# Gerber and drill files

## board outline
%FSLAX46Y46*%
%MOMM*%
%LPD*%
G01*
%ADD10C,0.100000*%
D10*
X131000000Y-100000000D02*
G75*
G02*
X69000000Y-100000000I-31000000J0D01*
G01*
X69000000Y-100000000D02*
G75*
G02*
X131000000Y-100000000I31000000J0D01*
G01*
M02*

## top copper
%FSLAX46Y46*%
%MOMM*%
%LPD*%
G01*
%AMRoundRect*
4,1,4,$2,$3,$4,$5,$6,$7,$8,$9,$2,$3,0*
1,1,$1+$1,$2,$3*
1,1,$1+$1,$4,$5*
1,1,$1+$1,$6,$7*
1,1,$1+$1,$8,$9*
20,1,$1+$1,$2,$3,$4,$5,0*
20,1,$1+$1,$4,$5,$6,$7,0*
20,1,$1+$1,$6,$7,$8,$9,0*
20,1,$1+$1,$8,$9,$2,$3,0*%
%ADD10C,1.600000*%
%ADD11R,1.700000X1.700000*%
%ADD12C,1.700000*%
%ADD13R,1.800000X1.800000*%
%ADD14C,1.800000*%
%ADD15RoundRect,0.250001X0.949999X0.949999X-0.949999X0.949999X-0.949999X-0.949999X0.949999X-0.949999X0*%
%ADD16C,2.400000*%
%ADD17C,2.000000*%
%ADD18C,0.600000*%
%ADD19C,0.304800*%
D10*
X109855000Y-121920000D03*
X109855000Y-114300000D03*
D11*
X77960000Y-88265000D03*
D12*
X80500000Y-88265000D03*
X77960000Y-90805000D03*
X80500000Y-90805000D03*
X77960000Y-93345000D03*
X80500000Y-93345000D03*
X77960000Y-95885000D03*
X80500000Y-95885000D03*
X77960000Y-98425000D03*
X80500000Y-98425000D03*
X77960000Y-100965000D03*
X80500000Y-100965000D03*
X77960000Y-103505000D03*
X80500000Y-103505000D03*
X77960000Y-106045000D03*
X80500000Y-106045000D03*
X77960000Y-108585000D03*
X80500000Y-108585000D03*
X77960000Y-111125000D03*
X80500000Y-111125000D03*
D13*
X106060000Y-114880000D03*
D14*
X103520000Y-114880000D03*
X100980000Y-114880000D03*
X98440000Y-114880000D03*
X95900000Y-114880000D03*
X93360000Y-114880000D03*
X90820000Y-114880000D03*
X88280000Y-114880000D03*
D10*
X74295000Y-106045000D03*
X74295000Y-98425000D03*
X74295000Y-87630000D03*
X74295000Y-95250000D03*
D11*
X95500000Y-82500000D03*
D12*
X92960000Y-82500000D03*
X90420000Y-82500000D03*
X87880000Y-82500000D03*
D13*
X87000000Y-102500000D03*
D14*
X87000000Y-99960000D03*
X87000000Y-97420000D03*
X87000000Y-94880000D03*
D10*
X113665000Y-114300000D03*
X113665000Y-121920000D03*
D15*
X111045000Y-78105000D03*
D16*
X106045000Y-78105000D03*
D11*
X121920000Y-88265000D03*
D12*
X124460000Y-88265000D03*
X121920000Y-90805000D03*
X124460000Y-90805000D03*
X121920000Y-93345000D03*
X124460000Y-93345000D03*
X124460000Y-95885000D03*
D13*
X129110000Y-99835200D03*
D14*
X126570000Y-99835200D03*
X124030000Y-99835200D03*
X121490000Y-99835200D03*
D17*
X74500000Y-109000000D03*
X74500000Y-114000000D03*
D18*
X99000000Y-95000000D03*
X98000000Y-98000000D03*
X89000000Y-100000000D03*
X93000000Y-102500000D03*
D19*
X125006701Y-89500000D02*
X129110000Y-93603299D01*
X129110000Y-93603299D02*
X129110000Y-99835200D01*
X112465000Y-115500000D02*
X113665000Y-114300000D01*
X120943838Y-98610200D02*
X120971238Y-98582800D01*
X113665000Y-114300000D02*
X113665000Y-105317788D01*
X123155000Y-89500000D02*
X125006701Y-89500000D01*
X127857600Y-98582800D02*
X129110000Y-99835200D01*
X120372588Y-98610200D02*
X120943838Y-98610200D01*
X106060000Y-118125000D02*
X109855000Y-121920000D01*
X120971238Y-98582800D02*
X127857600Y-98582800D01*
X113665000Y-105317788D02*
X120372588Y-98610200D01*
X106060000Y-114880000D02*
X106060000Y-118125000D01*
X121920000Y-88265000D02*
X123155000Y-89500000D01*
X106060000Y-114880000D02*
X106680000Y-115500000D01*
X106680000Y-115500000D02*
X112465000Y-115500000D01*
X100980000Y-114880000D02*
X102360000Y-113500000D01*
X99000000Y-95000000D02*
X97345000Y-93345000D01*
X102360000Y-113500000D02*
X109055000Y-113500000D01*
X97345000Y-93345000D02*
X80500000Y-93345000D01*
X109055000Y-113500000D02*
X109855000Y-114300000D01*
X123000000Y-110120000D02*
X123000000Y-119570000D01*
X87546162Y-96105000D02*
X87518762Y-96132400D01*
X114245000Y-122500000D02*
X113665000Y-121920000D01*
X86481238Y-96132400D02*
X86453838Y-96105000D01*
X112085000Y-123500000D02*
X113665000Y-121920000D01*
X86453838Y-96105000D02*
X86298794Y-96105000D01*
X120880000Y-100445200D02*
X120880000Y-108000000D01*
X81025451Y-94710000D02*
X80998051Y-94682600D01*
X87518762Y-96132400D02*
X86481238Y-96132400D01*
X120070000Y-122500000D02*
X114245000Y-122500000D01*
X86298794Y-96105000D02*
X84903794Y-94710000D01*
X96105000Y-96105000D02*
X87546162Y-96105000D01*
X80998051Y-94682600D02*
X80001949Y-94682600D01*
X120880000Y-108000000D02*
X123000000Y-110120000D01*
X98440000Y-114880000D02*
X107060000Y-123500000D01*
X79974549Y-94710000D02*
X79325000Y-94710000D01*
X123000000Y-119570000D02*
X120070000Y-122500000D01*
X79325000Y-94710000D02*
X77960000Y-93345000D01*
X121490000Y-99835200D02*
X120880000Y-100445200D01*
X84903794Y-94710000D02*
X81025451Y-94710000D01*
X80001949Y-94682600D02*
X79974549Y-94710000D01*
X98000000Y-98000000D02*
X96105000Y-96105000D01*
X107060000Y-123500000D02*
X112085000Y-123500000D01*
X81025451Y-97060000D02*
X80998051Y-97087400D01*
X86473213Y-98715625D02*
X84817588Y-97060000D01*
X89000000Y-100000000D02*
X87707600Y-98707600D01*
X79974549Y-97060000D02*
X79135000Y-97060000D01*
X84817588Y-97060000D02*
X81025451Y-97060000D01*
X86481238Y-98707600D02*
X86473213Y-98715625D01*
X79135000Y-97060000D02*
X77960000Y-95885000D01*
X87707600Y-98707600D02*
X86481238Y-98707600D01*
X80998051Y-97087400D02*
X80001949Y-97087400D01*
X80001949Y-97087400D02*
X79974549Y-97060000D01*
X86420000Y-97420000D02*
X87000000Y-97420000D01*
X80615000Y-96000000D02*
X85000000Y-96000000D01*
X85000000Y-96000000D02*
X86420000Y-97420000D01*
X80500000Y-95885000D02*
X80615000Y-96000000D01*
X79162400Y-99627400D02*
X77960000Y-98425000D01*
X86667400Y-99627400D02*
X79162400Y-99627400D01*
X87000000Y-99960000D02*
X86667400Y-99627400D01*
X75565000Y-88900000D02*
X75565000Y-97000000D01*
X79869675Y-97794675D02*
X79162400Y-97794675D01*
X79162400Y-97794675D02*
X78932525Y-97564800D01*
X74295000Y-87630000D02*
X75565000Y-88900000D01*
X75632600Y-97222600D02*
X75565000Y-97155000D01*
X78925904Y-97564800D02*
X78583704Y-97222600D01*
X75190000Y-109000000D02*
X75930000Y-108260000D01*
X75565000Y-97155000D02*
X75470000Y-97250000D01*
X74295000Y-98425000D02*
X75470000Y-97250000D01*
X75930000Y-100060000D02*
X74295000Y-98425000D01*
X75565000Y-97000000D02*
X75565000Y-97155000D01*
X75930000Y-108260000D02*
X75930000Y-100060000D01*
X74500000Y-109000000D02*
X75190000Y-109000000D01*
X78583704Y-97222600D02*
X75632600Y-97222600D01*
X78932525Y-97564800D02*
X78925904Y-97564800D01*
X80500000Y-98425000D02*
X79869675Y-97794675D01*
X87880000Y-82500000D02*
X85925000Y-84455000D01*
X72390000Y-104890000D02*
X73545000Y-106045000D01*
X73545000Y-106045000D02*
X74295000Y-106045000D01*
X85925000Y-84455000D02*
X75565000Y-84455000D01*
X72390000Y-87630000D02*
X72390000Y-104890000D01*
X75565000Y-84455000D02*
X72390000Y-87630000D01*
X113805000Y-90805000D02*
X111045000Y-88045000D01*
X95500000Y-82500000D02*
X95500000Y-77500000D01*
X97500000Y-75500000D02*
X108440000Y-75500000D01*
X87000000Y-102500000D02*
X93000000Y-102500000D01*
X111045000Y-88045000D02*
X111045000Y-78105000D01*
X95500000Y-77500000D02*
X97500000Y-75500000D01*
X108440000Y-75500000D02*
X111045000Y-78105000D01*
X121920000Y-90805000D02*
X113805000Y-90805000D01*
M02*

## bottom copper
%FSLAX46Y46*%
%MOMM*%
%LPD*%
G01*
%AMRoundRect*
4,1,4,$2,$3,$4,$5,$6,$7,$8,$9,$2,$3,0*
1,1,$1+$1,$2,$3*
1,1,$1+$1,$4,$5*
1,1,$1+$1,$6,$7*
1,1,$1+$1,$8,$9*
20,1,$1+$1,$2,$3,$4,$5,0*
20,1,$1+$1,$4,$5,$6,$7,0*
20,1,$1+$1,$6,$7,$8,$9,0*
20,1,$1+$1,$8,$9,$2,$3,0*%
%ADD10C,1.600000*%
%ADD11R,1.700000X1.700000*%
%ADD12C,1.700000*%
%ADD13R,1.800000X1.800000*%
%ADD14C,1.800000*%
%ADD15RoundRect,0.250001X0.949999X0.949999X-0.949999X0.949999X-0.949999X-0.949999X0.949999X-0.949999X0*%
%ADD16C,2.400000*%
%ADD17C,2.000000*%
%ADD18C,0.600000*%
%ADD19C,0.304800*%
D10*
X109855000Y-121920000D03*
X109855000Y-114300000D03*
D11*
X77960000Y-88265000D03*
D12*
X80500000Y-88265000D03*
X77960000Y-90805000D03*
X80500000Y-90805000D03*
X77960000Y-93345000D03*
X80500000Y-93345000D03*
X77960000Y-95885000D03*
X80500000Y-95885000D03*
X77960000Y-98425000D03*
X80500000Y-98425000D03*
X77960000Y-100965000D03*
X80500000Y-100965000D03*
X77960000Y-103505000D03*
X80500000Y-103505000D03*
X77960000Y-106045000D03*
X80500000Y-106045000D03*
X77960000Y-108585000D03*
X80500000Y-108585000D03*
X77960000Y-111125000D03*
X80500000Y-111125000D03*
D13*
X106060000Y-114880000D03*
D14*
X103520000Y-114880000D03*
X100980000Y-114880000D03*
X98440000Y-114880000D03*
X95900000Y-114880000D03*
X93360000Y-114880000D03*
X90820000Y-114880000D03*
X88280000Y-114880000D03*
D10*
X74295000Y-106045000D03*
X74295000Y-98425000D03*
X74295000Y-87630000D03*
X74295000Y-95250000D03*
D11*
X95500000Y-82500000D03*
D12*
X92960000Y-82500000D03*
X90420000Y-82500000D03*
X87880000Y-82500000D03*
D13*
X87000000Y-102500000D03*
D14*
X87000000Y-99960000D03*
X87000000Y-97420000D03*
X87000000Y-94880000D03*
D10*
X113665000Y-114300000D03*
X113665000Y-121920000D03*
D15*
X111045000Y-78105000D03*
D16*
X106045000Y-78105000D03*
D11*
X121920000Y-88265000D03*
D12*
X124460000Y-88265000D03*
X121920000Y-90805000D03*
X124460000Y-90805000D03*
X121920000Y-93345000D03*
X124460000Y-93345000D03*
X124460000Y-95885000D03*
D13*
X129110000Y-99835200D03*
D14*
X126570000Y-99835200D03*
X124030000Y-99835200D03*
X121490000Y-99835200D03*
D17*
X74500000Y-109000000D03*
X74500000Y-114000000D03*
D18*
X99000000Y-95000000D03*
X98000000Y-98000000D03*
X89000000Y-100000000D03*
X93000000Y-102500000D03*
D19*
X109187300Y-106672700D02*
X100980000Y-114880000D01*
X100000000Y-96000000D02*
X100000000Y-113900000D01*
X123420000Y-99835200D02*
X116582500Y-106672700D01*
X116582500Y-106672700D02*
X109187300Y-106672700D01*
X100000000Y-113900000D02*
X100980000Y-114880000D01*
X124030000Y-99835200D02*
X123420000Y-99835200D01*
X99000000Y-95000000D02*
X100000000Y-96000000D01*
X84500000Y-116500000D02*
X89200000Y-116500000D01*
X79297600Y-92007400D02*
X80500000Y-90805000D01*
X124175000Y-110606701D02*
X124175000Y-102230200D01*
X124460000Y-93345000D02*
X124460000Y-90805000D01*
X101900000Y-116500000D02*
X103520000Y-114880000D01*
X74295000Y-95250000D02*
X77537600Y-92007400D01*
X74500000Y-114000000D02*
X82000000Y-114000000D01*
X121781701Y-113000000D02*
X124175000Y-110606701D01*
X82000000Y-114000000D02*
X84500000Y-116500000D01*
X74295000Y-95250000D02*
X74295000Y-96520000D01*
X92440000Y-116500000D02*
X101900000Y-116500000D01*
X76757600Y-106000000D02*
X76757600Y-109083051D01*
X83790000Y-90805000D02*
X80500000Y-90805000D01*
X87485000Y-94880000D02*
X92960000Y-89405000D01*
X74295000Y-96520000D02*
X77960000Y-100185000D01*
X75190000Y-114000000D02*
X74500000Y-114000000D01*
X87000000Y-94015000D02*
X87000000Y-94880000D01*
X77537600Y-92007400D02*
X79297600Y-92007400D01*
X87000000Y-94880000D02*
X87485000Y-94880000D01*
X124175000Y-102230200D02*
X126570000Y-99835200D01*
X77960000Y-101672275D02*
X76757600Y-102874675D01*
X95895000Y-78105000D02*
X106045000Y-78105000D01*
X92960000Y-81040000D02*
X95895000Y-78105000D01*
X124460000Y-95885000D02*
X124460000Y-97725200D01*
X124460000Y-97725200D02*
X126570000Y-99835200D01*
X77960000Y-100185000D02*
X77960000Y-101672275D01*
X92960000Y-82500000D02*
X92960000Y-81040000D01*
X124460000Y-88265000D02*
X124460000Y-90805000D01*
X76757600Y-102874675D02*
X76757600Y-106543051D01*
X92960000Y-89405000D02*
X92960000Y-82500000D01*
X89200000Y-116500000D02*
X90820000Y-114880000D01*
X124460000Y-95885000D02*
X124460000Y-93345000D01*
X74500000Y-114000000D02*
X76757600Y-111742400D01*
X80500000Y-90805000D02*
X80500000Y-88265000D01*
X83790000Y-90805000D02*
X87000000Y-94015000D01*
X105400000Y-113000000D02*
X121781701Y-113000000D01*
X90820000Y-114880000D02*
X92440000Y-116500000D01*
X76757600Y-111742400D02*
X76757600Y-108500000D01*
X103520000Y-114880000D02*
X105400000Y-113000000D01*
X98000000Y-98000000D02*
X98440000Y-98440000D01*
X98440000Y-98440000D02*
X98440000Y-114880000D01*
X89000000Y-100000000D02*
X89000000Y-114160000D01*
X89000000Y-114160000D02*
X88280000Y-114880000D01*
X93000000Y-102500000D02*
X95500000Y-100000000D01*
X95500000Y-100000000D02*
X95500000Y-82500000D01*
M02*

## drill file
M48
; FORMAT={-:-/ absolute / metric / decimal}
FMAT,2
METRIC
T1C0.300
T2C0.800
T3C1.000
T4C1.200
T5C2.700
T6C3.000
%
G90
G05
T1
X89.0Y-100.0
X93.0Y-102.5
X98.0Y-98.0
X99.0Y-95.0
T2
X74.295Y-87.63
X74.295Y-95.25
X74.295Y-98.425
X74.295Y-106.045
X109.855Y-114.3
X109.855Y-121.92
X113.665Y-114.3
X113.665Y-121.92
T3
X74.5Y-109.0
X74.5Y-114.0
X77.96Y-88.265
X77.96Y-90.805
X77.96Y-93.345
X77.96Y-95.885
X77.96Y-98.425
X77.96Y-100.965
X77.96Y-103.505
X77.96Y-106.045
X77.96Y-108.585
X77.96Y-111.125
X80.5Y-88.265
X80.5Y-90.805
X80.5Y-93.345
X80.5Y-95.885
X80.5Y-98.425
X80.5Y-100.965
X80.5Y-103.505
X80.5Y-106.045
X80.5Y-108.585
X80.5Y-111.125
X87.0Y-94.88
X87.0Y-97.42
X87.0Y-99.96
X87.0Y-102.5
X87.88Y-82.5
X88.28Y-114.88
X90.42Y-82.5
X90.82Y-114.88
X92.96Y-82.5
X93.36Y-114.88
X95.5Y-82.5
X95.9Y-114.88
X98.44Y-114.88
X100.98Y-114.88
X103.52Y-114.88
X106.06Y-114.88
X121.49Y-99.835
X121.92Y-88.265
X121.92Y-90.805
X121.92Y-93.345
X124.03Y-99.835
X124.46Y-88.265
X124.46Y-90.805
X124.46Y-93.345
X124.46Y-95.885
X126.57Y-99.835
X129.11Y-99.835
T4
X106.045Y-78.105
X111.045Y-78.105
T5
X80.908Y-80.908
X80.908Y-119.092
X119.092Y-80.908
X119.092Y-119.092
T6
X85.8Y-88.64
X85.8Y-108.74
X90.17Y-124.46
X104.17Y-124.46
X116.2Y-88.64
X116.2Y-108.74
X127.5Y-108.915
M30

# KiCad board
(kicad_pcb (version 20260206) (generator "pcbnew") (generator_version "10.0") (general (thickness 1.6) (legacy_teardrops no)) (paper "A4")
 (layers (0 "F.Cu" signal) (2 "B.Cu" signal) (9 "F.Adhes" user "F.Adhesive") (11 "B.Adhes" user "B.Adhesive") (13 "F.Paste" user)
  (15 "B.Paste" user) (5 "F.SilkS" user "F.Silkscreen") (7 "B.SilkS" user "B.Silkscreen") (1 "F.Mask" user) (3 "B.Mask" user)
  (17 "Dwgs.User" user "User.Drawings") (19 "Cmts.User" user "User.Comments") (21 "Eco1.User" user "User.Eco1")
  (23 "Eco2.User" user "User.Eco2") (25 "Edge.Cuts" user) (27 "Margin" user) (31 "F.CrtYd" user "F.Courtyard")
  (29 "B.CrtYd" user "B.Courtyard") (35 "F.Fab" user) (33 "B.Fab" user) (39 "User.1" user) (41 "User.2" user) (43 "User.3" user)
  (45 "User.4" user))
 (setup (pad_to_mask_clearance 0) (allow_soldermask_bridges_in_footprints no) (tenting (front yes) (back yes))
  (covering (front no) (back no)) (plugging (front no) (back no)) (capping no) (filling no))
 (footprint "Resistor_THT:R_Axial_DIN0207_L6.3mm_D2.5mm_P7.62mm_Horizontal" (layer "F.Cu") (at 109.855 121.92 90)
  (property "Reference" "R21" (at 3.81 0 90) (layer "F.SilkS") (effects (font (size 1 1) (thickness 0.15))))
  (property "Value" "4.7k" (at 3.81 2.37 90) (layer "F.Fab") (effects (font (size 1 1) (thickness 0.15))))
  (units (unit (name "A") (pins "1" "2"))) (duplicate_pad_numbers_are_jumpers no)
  (pad "1" thru_hole circle (at 0 0 90) (size 1.6 1.6) (drill 0.8) (layers "*.Cu" "*.Mask") (remove_unused_layers no) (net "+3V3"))
  (pad "2" thru_hole circle (at 7.62 0 90) (size 1.6 1.6) (drill 0.8) (layers "*.Cu" "*.Mask") (remove_unused_layers no) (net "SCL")))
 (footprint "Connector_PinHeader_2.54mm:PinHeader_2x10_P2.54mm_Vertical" (layer "F.Cu") (at 77.96 88.265)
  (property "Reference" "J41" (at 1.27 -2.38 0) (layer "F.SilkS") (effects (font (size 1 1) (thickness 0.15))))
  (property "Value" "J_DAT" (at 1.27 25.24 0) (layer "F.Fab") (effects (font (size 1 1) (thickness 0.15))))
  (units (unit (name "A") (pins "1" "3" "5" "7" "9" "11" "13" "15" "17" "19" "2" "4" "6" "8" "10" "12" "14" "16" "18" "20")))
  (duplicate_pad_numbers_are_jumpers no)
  (pad "1" thru_hole rect (at 0 0) (size 1.7 1.7) (drill 1) (layers "*.Cu" "*.Mask") (remove_unused_layers no)
   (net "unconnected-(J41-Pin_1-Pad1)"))
  (pad "2" thru_hole circle (at 2.54 0) (size 1.7 1.7) (drill 1) (layers "*.Cu" "*.Mask") (remove_unused_layers no) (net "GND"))
  (pad "3" thru_hole circle (at 0 2.54) (size 1.7 1.7) (drill 1) (layers "*.Cu" "*.Mask") (remove_unused_layers no)
   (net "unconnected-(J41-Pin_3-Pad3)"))
  (pad "4" thru_hole circle (at 2.54 2.54) (size 1.7 1.7) (drill 1) (layers "*.Cu" "*.Mask") (remove_unused_layers no) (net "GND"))
  (pad "5" thru_hole circle (at 0 5.08) (size 1.7 1.7) (drill 1) (layers "*.Cu" "*.Mask") (remove_unused_layers no) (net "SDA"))
  (pad "6" thru_hole circle (at 2.54 5.08) (size 1.7 1.7) (drill 1) (layers "*.Cu" "*.Mask") (remove_unused_layers no) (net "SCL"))
  (pad "7" thru_hole circle (at 0 7.62) (size 1.7 1.7) (drill 1) (layers "*.Cu" "*.Mask") (remove_unused_layers no) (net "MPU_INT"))
  (pad "8" thru_hole circle (at 2.54 7.62) (size 1.7 1.7) (drill 1) (layers "*.Cu" "*.Mask") (remove_unused_layers no) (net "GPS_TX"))
  (pad "9" thru_hole circle (at 0 10.16) (size 1.7 1.7) (drill 1) (layers "*.Cu" "*.Mask") (remove_unused_layers no) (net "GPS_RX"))
  (pad "10" thru_hole circle (at 2.54 10.16) (size 1.7 1.7) (drill 1) (layers "*.Cu" "*.Mask") (remove_unused_layers no) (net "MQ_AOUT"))
  (pad "11" thru_hole circle (at 0 12.7) (size 1.7 1.7) (drill 1) (layers "*.Cu" "*.Mask") (remove_unused_layers no) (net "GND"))
  (pad "12" thru_hole circle (at 2.54 12.7) (size 1.7 1.7) (drill 1) (layers "*.Cu" "*.Mask") (remove_unused_layers no)
   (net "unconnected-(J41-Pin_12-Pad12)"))
  (pad "13" thru_hole circle (at 0 15.24) (size 1.7 1.7) (drill 1) (layers "*.Cu" "*.Mask") (remove_unused_layers no)
   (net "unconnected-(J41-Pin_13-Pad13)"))
  (pad "14" thru_hole circle (at 2.54 15.24) (size 1.7 1.7) (drill 1) (layers "*.Cu" "*.Mask") (remove_unused_layers no)
   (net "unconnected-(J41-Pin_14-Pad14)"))
  (pad "15" thru_hole circle (at 0 17.78) (size 1.7 1.7) (drill 1) (layers "*.Cu" "*.Mask") (remove_unused_layers no)
   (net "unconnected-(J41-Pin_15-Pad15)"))
  (pad "16" thru_hole circle (at 2.54 17.78) (size 1.7 1.7) (drill 1) (layers "*.Cu" "*.Mask") (remove_unused_layers no)
   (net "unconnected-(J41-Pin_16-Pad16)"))
  (pad "17" thru_hole circle (at 0 20.32) (size 1.7 1.7) (drill 1) (layers "*.Cu" "*.Mask") (remove_unused_layers no)
   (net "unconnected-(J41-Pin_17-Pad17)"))
  (pad "18" thru_hole circle (at 2.54 20.32) (size 1.7 1.7) (drill 1) (layers "*.Cu" "*.Mask") (remove_unused_layers no)
   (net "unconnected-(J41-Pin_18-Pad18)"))
  (pad "19" thru_hole circle (at 0 22.86) (size 1.7 1.7) (drill 1) (layers "*.Cu" "*.Mask") (remove_unused_layers no)
   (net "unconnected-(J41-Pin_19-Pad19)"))
  (pad "20" thru_hole circle (at 2.54 22.86) (size 1.7 1.7) (drill 1) (layers "*.Cu" "*.Mask") (remove_unused_layers no)
   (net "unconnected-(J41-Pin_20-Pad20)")))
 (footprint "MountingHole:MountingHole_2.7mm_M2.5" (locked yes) (layer "F.Cu") (at 119.092 119.092)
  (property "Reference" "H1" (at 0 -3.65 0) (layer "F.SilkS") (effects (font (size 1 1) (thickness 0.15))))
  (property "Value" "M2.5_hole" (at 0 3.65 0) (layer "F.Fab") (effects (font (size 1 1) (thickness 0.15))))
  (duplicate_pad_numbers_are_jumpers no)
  (pad "" np_thru_hole circle (at 0 0) (size 2.7 2.7) (drill 2.7) (layers "*.Cu" "*.Mask")))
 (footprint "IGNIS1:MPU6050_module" (layer "F.Cu") (at 97.17 119.96 -90)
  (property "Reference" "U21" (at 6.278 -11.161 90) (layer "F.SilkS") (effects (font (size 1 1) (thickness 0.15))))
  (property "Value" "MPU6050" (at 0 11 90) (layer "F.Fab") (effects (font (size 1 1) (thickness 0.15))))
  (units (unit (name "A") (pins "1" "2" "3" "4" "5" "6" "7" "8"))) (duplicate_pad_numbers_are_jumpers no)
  (pad "" np_thru_hole circle (at 4.5 -7 270) (size 3 3) (drill 3) (layers "*.Cu" "*.Mask"))
  (pad "" np_thru_hole circle (at 4.5 7 270) (size 3 3) (drill 3) (layers "*.Cu" "*.Mask"))
  (pad "1" thru_hole rect (at -5.08 -8.89 270) (size 1.8 1.8) (drill 1) (layers "*.Cu" "*.Mask") (remove_unused_layers no) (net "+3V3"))
  (pad "2" thru_hole circle (at -5.08 -6.35 270) (size 1.8 1.8) (drill 1) (layers "*.Cu" "*.Mask") (remove_unused_layers no) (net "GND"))
  (pad "3" thru_hole circle (at -5.08 -3.81 270) (size 1.8 1.8) (drill 1) (layers "*.Cu" "*.Mask") (remove_unused_layers no) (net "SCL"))
  (pad "4" thru_hole circle (at -5.08 -1.27 270) (size 1.8 1.8) (drill 1) (layers "*.Cu" "*.Mask") (remove_unused_layers no) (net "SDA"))
  (pad "5" thru_hole circle (at -5.08 1.27 270) (size 1.8 1.8) (drill 1) (layers "*.Cu" "*.Mask") (remove_unused_layers no)
   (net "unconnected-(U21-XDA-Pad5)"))
  (pad "6" thru_hole circle (at -5.08 3.81 270) (size 1.8 1.8) (drill 1) (layers "*.Cu" "*.Mask") (remove_unused_layers no)
   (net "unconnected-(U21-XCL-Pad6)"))
  (pad "7" thru_hole circle (at -5.08 6.35 270) (size 1.8 1.8) (drill 1) (layers "*.Cu" "*.Mask") (remove_unused_layers no) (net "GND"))
  (pad "8" thru_hole circle (at -5.08 8.89 270) (size 1.8 1.8) (drill 1) (layers "*.Cu" "*.Mask") (remove_unused_layers no) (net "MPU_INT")))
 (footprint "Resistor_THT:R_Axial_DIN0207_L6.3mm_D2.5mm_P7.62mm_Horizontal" (layer "F.Cu") (at 74.295 106.045 90)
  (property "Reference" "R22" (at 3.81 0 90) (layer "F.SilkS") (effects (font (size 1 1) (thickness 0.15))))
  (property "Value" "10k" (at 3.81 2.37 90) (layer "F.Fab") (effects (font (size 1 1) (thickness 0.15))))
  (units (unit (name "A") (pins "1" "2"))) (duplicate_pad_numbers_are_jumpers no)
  (pad "1" thru_hole circle (at 0 0 90) (size 1.6 1.6) (drill 0.8) (layers "*.Cu" "*.Mask") (remove_unused_layers no) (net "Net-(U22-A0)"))
  (pad "2" thru_hole circle (at 7.62 0 90) (size 1.6 1.6) (drill 0.8) (layers "*.Cu" "*.Mask") (remove_unused_layers no) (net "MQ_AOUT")))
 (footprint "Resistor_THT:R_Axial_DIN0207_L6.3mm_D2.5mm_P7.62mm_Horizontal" (layer "F.Cu") (at 74.295 87.63 -90)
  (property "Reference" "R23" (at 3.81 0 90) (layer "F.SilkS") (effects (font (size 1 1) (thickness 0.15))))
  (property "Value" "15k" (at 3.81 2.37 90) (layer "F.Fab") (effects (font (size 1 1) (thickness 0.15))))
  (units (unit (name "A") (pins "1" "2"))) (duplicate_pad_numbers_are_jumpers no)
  (pad "1" thru_hole circle (at 0 0 270) (size 1.6 1.6) (drill 0.8) (layers "*.Cu" "*.Mask") (remove_unused_layers no) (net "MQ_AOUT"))
  (pad "2" thru_hole circle (at 7.62 0 270) (size 1.6 1.6) (drill 0.8) (layers "*.Cu" "*.Mask") (remove_unused_layers no) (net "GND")))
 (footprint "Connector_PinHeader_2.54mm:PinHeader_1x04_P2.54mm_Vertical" (layer "F.Cu") (at 95.5 82.5 -90)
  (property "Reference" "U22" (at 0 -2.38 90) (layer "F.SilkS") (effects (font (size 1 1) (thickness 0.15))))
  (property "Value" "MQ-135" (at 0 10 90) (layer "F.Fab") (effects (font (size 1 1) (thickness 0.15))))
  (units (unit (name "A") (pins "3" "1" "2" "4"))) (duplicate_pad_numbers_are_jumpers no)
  (pad "1" thru_hole rect (at 0 0 270) (size 1.7 1.7) (drill 1) (layers "*.Cu" "*.Mask") (remove_unused_layers no) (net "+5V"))
  (pad "2" thru_hole circle (at 0 2.54 270) (size 1.7 1.7) (drill 1) (layers "*.Cu" "*.Mask") (remove_unused_layers no) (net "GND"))
  (pad "3" thru_hole circle (at 0 5.08 270) (size 1.7 1.7) (drill 1) (layers "*.Cu" "*.Mask") (remove_unused_layers no)
   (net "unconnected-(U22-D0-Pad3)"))
  (pad "4" thru_hole circle (at 0 7.62 270) (size 1.7 1.7) (drill 1) (layers "*.Cu" "*.Mask") (remove_unused_layers no) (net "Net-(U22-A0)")))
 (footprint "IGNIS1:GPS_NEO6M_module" (layer "F.Cu") (at 101 98.69)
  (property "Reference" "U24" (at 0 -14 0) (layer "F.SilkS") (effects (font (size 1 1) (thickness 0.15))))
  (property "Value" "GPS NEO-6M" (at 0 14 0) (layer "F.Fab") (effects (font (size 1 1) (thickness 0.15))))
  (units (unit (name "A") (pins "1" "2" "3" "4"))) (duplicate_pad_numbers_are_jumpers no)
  (pad "" np_thru_hole circle (at -15.2 -10.05) (size 3 3) (drill 3) (layers "*.Cu" "*.Mask"))
  (pad "" np_thru_hole circle (at -15.2 10.05) (size 3 3) (drill 3) (layers "*.Cu" "*.Mask"))
  (pad "" np_thru_hole circle (at 15.2 -10.05) (size 3 3) (drill 3) (layers "*.Cu" "*.Mask"))
  (pad "" np_thru_hole circle (at 15.2 10.05) (size 3 3) (drill 3) (layers "*.Cu" "*.Mask"))
  (pad "1" thru_hole rect (at -14 3.81) (size 1.8 1.8) (drill 1) (layers "*.Cu" "*.Mask") (remove_unused_layers no) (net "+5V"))
  (pad "2" thru_hole circle (at -14 1.27) (size 1.8 1.8) (drill 1) (layers "*.Cu" "*.Mask") (remove_unused_layers no) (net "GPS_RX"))
  (pad "3" thru_hole circle (at -14 -1.27) (size 1.8 1.8) (drill 1) (layers "*.Cu" "*.Mask") (remove_unused_layers no) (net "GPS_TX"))
  (pad "4" thru_hole circle (at -14 -3.81) (size 1.8 1.8) (drill 1) (layers "*.Cu" "*.Mask") (remove_unused_layers no) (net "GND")))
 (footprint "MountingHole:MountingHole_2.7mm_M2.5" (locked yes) (layer "F.Cu") (at 80.908 80.908)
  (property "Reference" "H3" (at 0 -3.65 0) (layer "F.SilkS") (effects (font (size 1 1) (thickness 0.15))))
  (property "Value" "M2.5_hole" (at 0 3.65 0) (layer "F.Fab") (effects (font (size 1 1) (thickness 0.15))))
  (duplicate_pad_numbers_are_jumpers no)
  (pad "" np_thru_hole circle (at 0 0) (size 2.7 2.7) (drill 2.7) (layers "*.Cu" "*.Mask")))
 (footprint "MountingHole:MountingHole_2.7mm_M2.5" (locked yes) (layer "F.Cu") (at 119.092 80.908)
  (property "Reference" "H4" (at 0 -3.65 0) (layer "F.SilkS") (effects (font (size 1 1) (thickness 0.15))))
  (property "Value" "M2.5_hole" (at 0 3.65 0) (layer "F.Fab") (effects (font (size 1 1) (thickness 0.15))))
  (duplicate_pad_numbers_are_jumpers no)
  (pad "" np_thru_hole circle (at 0 0) (size 2.7 2.7) (drill 2.7) (layers "*.Cu" "*.Mask")))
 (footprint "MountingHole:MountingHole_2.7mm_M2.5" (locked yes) (layer "F.Cu") (at 80.908 119.092)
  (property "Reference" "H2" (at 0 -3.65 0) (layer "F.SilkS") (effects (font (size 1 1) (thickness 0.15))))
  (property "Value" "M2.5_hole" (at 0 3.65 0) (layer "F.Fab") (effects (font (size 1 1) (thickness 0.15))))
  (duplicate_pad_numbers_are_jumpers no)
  (pad "" np_thru_hole circle (at 0 0) (size 2.7 2.7) (drill 2.7) (layers "*.Cu" "*.Mask")))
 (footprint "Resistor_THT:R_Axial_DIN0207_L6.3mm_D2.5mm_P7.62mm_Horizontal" (layer "F.Cu") (at 113.665 114.3 -90)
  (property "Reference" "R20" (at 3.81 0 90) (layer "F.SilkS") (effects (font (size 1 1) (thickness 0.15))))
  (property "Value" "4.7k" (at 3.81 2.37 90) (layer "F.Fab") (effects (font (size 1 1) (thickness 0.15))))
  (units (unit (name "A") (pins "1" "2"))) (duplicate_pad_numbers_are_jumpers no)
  (pad "1" thru_hole circle (at 0 0 270) (size 1.6 1.6) (drill 0.8) (layers "*.Cu" "*.Mask") (remove_unused_layers no) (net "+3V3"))
  (pad "2" thru_hole circle (at 7.62 0 270) (size 1.6 1.6) (drill 0.8) (layers "*.Cu" "*.Mask") (remove_unused_layers no) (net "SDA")))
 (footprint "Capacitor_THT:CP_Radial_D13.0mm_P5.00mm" (layer "F.Cu") (at 111.045 78.105 180)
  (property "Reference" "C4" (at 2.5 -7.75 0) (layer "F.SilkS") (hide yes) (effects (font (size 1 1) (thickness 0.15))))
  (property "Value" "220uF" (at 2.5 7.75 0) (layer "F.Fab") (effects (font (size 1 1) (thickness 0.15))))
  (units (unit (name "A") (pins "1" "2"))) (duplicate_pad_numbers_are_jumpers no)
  (pad "1" thru_hole roundrect (at 0 0 180) (size 2.4 2.4) (drill 1.2) (layers "*.Cu" "*.Mask") (remove_unused_layers no)
   (roundrect_rratio 0.104167) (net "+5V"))
  (pad "2" thru_hole circle (at 5 0 180) (size 2.4 2.4) (drill 1.2) (layers "*.Cu" "*.Mask") (remove_unused_layers no) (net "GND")))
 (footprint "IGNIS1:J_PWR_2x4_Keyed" (layer "F.Cu") (at 123.19 92.075)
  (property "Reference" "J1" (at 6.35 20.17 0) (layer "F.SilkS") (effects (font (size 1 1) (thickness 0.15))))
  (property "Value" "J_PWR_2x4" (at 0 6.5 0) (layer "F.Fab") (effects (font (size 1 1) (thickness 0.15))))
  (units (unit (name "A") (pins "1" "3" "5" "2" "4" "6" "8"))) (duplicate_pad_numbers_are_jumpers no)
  (pad "1" thru_hole rect (at -1.27 -3.81) (size 1.7 1.7) (drill 1) (layers "*.Cu" "*.Mask") (remove_unused_layers no) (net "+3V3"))
  (pad "2" thru_hole circle (at 1.27 -3.81) (size 1.7 1.7) (drill 1) (layers "*.Cu" "*.Mask") (remove_unused_layers no) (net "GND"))
  (pad "3" thru_hole circle (at -1.27 -1.27) (size 1.7 1.7) (drill 1) (layers "*.Cu" "*.Mask") (remove_unused_layers no) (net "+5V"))
  (pad "4" thru_hole circle (at 1.27 -1.27) (size 1.7 1.7) (drill 1) (layers "*.Cu" "*.Mask") (remove_unused_layers no) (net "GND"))
  (pad "5" thru_hole circle (at -1.27 1.27) (size 1.7 1.7) (drill 1) (layers "*.Cu" "*.Mask") (remove_unused_layers no)
   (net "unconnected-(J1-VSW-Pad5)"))
  (pad "6" thru_hole circle (at 1.27 1.27) (size 1.7 1.7) (drill 1) (layers "*.Cu" "*.Mask") (remove_unused_layers no) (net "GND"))
  (pad "8" thru_hole circle (at 1.27 3.81) (size 1.7 1.7) (drill 1) (layers "*.Cu" "*.Mask") (remove_unused_layers no) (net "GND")))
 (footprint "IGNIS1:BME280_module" (layer "F.Cu") (at 125.3 104.9152 -90)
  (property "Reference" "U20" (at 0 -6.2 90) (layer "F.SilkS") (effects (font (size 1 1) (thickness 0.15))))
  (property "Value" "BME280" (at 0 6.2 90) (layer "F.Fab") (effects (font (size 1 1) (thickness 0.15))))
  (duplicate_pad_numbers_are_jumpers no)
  (pad "" np_thru_hole circle (at 4 -2.2 270) (size 3 3) (drill 3) (layers "*.Cu" "*.Mask"))
  (pad "1" thru_hole rect (at -5.08 -3.81 270) (size 1.8 1.8) (drill 1) (layers "*.Cu" "*.Mask") (remove_unused_layers no) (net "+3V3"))
  (pad "2" thru_hole circle (at -5.08 -1.27 270) (size 1.8 1.8) (drill 1) (layers "*.Cu" "*.Mask") (remove_unused_layers no) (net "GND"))
  (pad "3" thru_hole circle (at -5.08 1.27 270) (size 1.8 1.8) (drill 1) (layers "*.Cu" "*.Mask") (remove_unused_layers no) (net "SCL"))
  (pad "4" thru_hole circle (at -5.08 3.81 270) (size 1.8 1.8) (drill 1) (layers "*.Cu" "*.Mask") (remove_unused_layers no) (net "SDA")))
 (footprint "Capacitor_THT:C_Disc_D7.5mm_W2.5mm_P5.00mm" (layer "F.Cu") (at 74.5 109 -90)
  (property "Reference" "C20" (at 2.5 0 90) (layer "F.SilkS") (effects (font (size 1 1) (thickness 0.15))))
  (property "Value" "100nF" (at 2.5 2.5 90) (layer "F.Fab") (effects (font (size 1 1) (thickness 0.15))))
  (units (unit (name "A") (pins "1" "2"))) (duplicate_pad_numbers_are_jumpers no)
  (pad "1" thru_hole circle (at 0 0 270) (size 2 2) (drill 1) (layers "*.Cu" "*.Mask") (remove_unused_layers no) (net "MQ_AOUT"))
  (pad "2" thru_hole circle (at 5 0 270) (size 2 2) (drill 1) (layers "*.Cu" "*.Mask") (remove_unused_layers no) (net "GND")))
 (gr_circle (center 100 100) (end 131 100) (stroke (width 0.1) (type solid)) (fill no) (locked yes) (layer "Edge.Cuts"))
 (segment (start 125.006701 89.5) (end 129.11 93.603299) (width 0.3048) (layer "F.Cu") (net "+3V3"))
 (segment (start 129.11 93.603299) (end 129.11 99.8352) (width 0.3048) (layer "F.Cu") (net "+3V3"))
 (segment (start 112.465 115.5) (end 113.665 114.3) (width 0.3048) (layer "F.Cu") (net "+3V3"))
 (segment (start 120.943838 98.6102) (end 120.971238 98.5828) (width 0.3048) (layer "F.Cu") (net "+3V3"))
 (segment (start 113.665 114.3) (end 113.665 105.317788) (width 0.3048) (layer "F.Cu") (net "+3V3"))
 (segment (start 123.155 89.5) (end 125.006701 89.5) (width 0.3048) (layer "F.Cu") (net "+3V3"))
 (segment (start 127.8576 98.5828) (end 129.11 99.8352) (width 0.3048) (layer "F.Cu") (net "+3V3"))
 (segment (start 120.372588 98.6102) (end 120.943838 98.6102) (width 0.3048) (layer "F.Cu") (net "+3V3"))
 (segment (start 106.06 118.125) (end 109.855 121.92) (width 0.3048) (layer "F.Cu") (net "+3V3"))
 (segment (start 120.971238 98.5828) (end 127.8576 98.5828) (width 0.3048) (layer "F.Cu") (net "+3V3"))
 (segment (start 113.665 105.317788) (end 120.372588 98.6102) (width 0.3048) (layer "F.Cu") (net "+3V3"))
 (segment (start 106.06 114.88) (end 106.06 118.125) (width 0.3048) (layer "F.Cu") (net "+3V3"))
 (segment (start 121.92 88.265) (end 123.155 89.5) (width 0.3048) (layer "F.Cu") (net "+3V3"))
 (segment (start 106.06 114.88) (end 106.68 115.5) (width 0.3048) (layer "F.Cu") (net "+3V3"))
 (segment (start 106.68 115.5) (end 112.465 115.5) (width 0.3048) (layer "F.Cu") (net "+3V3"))
 (segment (start 100.98 114.88) (end 102.36 113.5) (width 0.3048) (layer "F.Cu") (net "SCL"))
 (segment (start 99 95) (end 97.345 93.345) (width 0.3048) (layer "F.Cu") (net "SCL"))
 (segment (start 102.36 113.5) (end 109.055 113.5) (width 0.3048) (layer "F.Cu") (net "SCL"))
 (segment (start 97.345 93.345) (end 80.5 93.345) (width 0.3048) (layer "F.Cu") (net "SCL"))
 (segment (start 109.055 113.5) (end 109.855 114.3) (width 0.3048) (layer "F.Cu") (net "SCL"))
 (via (at 99 95) (size 0.6) (drill 0.3) (layers "F.Cu" "B.Cu") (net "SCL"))
 (segment (start 109.1873 106.6727) (end 100.98 114.88) (width 0.3048) (layer "B.Cu") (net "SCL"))
 (segment (start 100 96) (end 100 113.9) (width 0.3048) (layer "B.Cu") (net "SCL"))
 (segment (start 123.42 99.8352) (end 116.5825 106.6727) (width 0.3048) (layer "B.Cu") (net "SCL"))
 (segment (start 116.5825 106.6727) (end 109.1873 106.6727) (width 0.3048) (layer "B.Cu") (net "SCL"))
 (segment (start 100 113.9) (end 100.98 114.88) (width 0.3048) (layer "B.Cu") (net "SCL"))
 (segment (start 124.03 99.8352) (end 123.42 99.8352) (width 0.3048) (layer "B.Cu") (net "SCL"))
 (segment (start 99 95) (end 100 96) (width 0.3048) (layer "B.Cu") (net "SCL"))
 (segment (start 84.5 116.5) (end 89.2 116.5) (width 0.3048) (layer "B.Cu") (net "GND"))
 (segment (start 79.2976 92.0074) (end 80.5 90.805) (width 0.3048) (layer "B.Cu") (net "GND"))
 (segment (start 124.175 110.606701) (end 124.175 102.2302) (width 0.3048) (layer "B.Cu") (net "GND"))
 (segment (start 124.46 93.345) (end 124.46 90.805) (width 0.3048) (layer "B.Cu") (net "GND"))
 (segment (start 101.9 116.5) (end 103.52 114.88) (width 0.3048) (layer "B.Cu") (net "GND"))
 (segment (start 74.295 95.25) (end 77.5376 92.0074) (width 0.3048) (layer "B.Cu") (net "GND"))
 (segment (start 74.5 114) (end 82 114) (width 0.3048) (layer "B.Cu") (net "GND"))
 (segment (start 121.781701 113) (end 124.175 110.606701) (width 0.3048) (layer "B.Cu") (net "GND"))
 (segment (start 82 114) (end 84.5 116.5) (width 0.3048) (layer "B.Cu") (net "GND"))
 (segment (start 74.295 95.25) (end 74.295 96.52) (width 0.3048) (layer "B.Cu") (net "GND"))
 (segment (start 92.44 116.5) (end 101.9 116.5) (width 0.3048) (layer "B.Cu") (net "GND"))
 (segment (start 76.7576 106) (end 76.7576 109.083051) (width 0.3048) (layer "B.Cu") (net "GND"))
 (segment (start 83.79 90.805) (end 80.5 90.805) (width 0.3048) (layer "B.Cu") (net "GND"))
 (segment (start 87.485 94.88) (end 92.96 89.405) (width 0.3048) (layer "B.Cu") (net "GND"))
 (segment (start 74.295 96.52) (end 77.96 100.185) (width 0.3048) (layer "B.Cu") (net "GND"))
 (segment (start 75.19 114) (end 74.5 114) (width 0.3048) (layer "B.Cu") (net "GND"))
 (segment (start 87 94.015) (end 87 94.88) (width 0.3048) (layer "B.Cu") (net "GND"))
 (segment (start 77.5376 92.0074) (end 79.2976 92.0074) (width 0.3048) (layer "B.Cu") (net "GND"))
 (segment (start 87 94.88) (end 87.485 94.88) (width 0.3048) (layer "B.Cu") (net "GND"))
 (segment (start 124.175 102.2302) (end 126.57 99.8352) (width 0.3048) (layer "B.Cu") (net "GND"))
 (segment (start 77.96 101.672275) (end 76.7576 102.874675) (width 0.3048) (layer "B.Cu") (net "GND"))
 (segment (start 95.895 78.105) (end 106.045 78.105) (width 0.3048) (layer "B.Cu") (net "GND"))
 (segment (start 92.96 81.04) (end 95.895 78.105) (width 0.3048) (layer "B.Cu") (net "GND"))
 (segment (start 124.46 95.885) (end 124.46 97.7252) (width 0.3048) (layer "B.Cu") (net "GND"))
 (segment (start 124.46 97.7252) (end 126.57 99.8352) (width 0.3048) (layer "B.Cu") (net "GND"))
 (segment (start 77.96 100.185) (end 77.96 101.672275) (width 0.3048) (layer "B.Cu") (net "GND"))
 (segment (start 92.96 82.5) (end 92.96 81.04) (width 0.3048) (layer "B.Cu") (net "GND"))
 (segment (start 124.46 88.265) (end 124.46 90.805) (width 0.3048) (layer "B.Cu") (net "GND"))
 (segment (start 76.7576 102.874675) (end 76.7576 106.543051) (width 0.3048) (layer "B.Cu") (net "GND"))
 (segment (start 92.96 89.405) (end 92.96 82.5) (width 0.3048) (layer "B.Cu") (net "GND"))
 (segment (start 89.2 116.5) (end 90.82 114.88) (width 0.3048) (layer "B.Cu") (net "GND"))
 (segment (start 124.46 95.885) (end 124.46 93.345) (width 0.3048) (layer "B.Cu") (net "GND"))
 (segment (start 74.5 114) (end 76.7576 111.7424) (width 0.3048) (layer "B.Cu") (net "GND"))
 (segment (start 80.5 90.805) (end 80.5 88.265) (width 0.3048) (layer "B.Cu") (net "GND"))
 (segment (start 83.79 90.805) (end 87 94.015) (width 0.3048) (layer "B.Cu") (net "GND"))
 (segment (start 105.4 113) (end 121.781701 113) (width 0.3048) (layer "B.Cu") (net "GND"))
 (segment (start 90.82 114.88) (end 92.44 116.5) (width 0.3048) (layer "B.Cu") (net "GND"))
 (segment (start 76.7576 111.7424) (end 76.7576 108.5) (width 0.3048) (layer "B.Cu") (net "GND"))
 (segment (start 103.52 114.88) (end 105.4 113) (width 0.3048) (layer "B.Cu") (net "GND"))
 (segment (start 123 110.12) (end 123 119.57) (width 0.3048) (layer "F.Cu") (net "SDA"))
 (segment (start 87.546162 96.105) (end 87.518762 96.1324) (width 0.3048) (layer "F.Cu") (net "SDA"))
 (segment (start 114.245 122.5) (end 113.665 121.92) (width 0.3048) (layer "F.Cu") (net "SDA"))
 (segment (start 86.481238 96.1324) (end 86.453838 96.105) (width 0.3048) (layer "F.Cu") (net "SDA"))
 (segment (start 112.085 123.5) (end 113.665 121.92) (width 0.3048) (layer "F.Cu") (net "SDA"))
 (segment (start 86.453838 96.105) (end 86.298794 96.105) (width 0.3048) (layer "F.Cu") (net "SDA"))
 (segment (start 120.88 100.4452) (end 120.88 108) (width 0.3048) (layer "F.Cu") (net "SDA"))
 (segment (start 81.025451 94.71) (end 80.998051 94.6826) (width 0.3048) (layer "F.Cu") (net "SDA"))
 (segment (start 87.518762 96.1324) (end 86.481238 96.1324) (width 0.3048) (layer "F.Cu") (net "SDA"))
 (segment (start 120.07 122.5) (end 114.245 122.5) (width 0.3048) (layer "F.Cu") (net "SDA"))
 (segment (start 86.298794 96.105) (end 84.903794 94.71) (width 0.3048) (layer "F.Cu") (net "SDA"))
 (segment (start 96.105 96.105) (end 87.546162 96.105) (width 0.3048) (layer "F.Cu") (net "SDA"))
 (segment (start 80.998051 94.6826) (end 80.001949 94.6826) (width 0.3048) (layer "F.Cu") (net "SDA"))
 (segment (start 120.88 108) (end 123 110.12) (width 0.3048) (layer "F.Cu") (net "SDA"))
 (segment (start 98.44 114.88) (end 107.06 123.5) (width 0.3048) (layer "F.Cu") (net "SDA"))
 (segment (start 79.974549 94.71) (end 79.325 94.71) (width 0.3048) (layer "F.Cu") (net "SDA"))
 (segment (start 123 119.57) (end 120.07 122.5) (width 0.3048) (layer "F.Cu") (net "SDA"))
 (segment (start 79.325 94.71) (end 77.96 93.345) (width 0.3048) (layer "F.Cu") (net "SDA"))
 (segment (start 121.49 99.8352) (end 120.88 100.4452) (width 0.3048) (layer "F.Cu") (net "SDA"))
 (segment (start 84.903794 94.71) (end 81.025451 94.71) (width 0.3048) (layer "F.Cu") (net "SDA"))
 (segment (start 80.001949 94.6826) (end 79.974549 94.71) (width 0.3048) (layer "F.Cu") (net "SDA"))
 (segment (start 98 98) (end 96.105 96.105) (width 0.3048) (layer "F.Cu") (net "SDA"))
 (segment (start 107.06 123.5) (end 112.085 123.5) (width 0.3048) (layer "F.Cu") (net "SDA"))
 (via (at 98 98) (size 0.6) (drill 0.3) (layers "F.Cu" "B.Cu") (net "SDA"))
 (segment (start 98 98) (end 98.44 98.44) (width 0.3048) (layer "B.Cu") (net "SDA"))
 (segment (start 98.44 98.44) (end 98.44 114.88) (width 0.3048) (layer "B.Cu") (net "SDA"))
 (segment (start 81.025451 97.06) (end 80.998051 97.0874) (width 0.3048) (layer "F.Cu") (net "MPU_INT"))
 (segment (start 86.473213 98.715625) (end 84.817588 97.06) (width 0.3048) (layer "F.Cu") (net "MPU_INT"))
 (segment (start 89 100) (end 87.7076 98.7076) (width 0.3048) (layer "F.Cu") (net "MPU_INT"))
 (segment (start 79.974549 97.06) (end 79.135 97.06) (width 0.3048) (layer "F.Cu") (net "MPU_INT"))
 (segment (start 84.817588 97.06) (end 81.025451 97.06) (width 0.3048) (layer "F.Cu") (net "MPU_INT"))
 (segment (start 86.481238 98.7076) (end 86.473213 98.715625) (width 0.3048) (layer "F.Cu") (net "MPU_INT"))
 (segment (start 79.135 97.06) (end 77.96 95.885) (width 0.3048) (layer "F.Cu") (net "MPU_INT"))
 (segment (start 87.7076 98.7076) (end 86.481238 98.7076) (width 0.3048) (layer "F.Cu") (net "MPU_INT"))
 (segment (start 80.998051 97.0874) (end 80.001949 97.0874) (width 0.3048) (layer "F.Cu") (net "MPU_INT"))
 (segment (start 80.001949 97.0874) (end 79.974549 97.06) (width 0.3048) (layer "F.Cu") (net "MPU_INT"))
 (via (at 89 100) (size 0.6) (drill 0.3) (layers "F.Cu" "B.Cu") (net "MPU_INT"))
 (segment (start 89 100) (end 89 114.16) (width 0.3048) (layer "B.Cu") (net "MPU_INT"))
 (segment (start 89 114.16) (end 88.28 114.88) (width 0.3048) (layer "B.Cu") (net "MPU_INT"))
 (segment (start 86.42 97.42) (end 87 97.42) (width 0.3048) (layer "F.Cu") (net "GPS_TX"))
 (segment (start 80.615 96) (end 85 96) (width 0.3048) (layer "F.Cu") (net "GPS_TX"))
 (segment (start 85 96) (end 86.42 97.42) (width 0.3048) (layer "F.Cu") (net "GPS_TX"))
 (segment (start 80.5 95.885) (end 80.615 96) (width 0.3048) (layer "F.Cu") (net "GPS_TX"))
 (segment (start 79.1624 99.6274) (end 77.96 98.425) (width 0.3048) (layer "F.Cu") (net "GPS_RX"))
 (segment (start 86.6674 99.6274) (end 79.1624 99.6274) (width 0.3048) (layer "F.Cu") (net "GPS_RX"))
 (segment (start 87 99.96) (end 86.6674 99.6274) (width 0.3048) (layer "F.Cu") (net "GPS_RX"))
 (segment (start 75.565 88.9) (end 75.565 97) (width 0.3048) (layer "F.Cu") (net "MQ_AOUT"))
 (segment (start 79.869675 97.794675) (end 79.1624 97.794675) (width 0.3048) (layer "F.Cu") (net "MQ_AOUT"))
 (segment (start 79.1624 97.794675) (end 78.932525 97.5648) (width 0.3048) (layer "F.Cu") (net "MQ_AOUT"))
 (segment (start 74.295 87.63) (end 75.565 88.9) (width 0.3048) (layer "F.Cu") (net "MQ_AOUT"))
 (segment (start 75.6326 97.2226) (end 75.565 97.155) (width 0.3048) (layer "F.Cu") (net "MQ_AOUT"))
 (segment (start 78.925904 97.5648) (end 78.583704 97.2226) (width 0.3048) (layer "F.Cu") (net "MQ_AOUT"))
 (segment (start 75.19 109) (end 75.93 108.26) (width 0.3048) (layer "F.Cu") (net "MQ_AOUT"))
 (segment (start 75.565 97.155) (end 75.47 97.25) (width 0.3048) (layer "F.Cu") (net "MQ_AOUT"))
 (segment (start 74.295 98.425) (end 75.47 97.25) (width 0.3048) (layer "F.Cu") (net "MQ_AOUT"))
 (segment (start 75.93 100.06) (end 74.295 98.425) (width 0.3048) (layer "F.Cu") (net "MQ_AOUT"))
 (segment (start 75.565 97) (end 75.565 97.155) (width 0.3048) (layer "F.Cu") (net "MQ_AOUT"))
 (segment (start 75.93 108.26) (end 75.93 100.06) (width 0.3048) (layer "F.Cu") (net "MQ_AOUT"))
 (segment (start 74.5 109) (end 75.19 109) (width 0.3048) (layer "F.Cu") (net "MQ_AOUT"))
 (segment (start 78.583704 97.2226) (end 75.6326 97.2226) (width 0.3048) (layer "F.Cu") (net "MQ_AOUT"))
 (segment (start 78.932525 97.5648) (end 78.925904 97.5648) (width 0.3048) (layer "F.Cu") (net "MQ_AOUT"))
 (segment (start 80.5 98.425) (end 79.869675 97.794675) (width 0.3048) (layer "F.Cu") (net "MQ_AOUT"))
 (segment (start 87.88 82.5) (end 85.925 84.455) (width 0.3048) (layer "F.Cu") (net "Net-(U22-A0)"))
 (segment (start 72.39 104.89) (end 73.545 106.045) (width 0.3048) (layer "F.Cu") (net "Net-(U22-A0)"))
 (segment (start 73.545 106.045) (end 74.295 106.045) (width 0.3048) (layer "F.Cu") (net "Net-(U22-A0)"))
 (segment (start 85.925 84.455) (end 75.565 84.455) (width 0.3048) (layer "F.Cu") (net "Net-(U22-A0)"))
 (segment (start 72.39 87.63) (end 72.39 104.89) (width 0.3048) (layer "F.Cu") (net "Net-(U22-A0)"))
 (segment (start 75.565 84.455) (end 72.39 87.63) (width 0.3048) (layer "F.Cu") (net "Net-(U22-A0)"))
 (segment (start 113.805 90.805) (end 111.045 88.045) (width 0.3048) (layer "F.Cu") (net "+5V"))
 (segment (start 95.5 82.5) (end 95.5 77.5) (width 0.3048) (layer "F.Cu") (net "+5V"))
 (segment (start 97.5 75.5) (end 108.44 75.5) (width 0.3048) (layer "F.Cu") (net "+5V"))
 (segment (start 87 102.5) (end 93 102.5) (width 0.3048) (layer "F.Cu") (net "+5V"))
 (segment (start 111.045 88.045) (end 111.045 78.105) (width 0.3048) (layer "F.Cu") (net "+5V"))
 (segment (start 95.5 77.5) (end 97.5 75.5) (width 0.3048) (layer "F.Cu") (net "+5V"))
 (segment (start 108.44 75.5) (end 111.045 78.105) (width 0.3048) (layer "F.Cu") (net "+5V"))
 (segment (start 121.92 90.805) (end 113.805 90.805) (width 0.3048) (layer "F.Cu") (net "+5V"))
 (via (at 93 102.5) (size 0.6) (drill 0.3) (layers "F.Cu" "B.Cu") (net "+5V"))
 (segment (start 93 102.5) (end 95.5 100) (width 0.3048) (layer "B.Cu") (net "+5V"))
 (segment (start 95.5 100) (end 95.5 82.5) (width 0.3048) (layer "B.Cu") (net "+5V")))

